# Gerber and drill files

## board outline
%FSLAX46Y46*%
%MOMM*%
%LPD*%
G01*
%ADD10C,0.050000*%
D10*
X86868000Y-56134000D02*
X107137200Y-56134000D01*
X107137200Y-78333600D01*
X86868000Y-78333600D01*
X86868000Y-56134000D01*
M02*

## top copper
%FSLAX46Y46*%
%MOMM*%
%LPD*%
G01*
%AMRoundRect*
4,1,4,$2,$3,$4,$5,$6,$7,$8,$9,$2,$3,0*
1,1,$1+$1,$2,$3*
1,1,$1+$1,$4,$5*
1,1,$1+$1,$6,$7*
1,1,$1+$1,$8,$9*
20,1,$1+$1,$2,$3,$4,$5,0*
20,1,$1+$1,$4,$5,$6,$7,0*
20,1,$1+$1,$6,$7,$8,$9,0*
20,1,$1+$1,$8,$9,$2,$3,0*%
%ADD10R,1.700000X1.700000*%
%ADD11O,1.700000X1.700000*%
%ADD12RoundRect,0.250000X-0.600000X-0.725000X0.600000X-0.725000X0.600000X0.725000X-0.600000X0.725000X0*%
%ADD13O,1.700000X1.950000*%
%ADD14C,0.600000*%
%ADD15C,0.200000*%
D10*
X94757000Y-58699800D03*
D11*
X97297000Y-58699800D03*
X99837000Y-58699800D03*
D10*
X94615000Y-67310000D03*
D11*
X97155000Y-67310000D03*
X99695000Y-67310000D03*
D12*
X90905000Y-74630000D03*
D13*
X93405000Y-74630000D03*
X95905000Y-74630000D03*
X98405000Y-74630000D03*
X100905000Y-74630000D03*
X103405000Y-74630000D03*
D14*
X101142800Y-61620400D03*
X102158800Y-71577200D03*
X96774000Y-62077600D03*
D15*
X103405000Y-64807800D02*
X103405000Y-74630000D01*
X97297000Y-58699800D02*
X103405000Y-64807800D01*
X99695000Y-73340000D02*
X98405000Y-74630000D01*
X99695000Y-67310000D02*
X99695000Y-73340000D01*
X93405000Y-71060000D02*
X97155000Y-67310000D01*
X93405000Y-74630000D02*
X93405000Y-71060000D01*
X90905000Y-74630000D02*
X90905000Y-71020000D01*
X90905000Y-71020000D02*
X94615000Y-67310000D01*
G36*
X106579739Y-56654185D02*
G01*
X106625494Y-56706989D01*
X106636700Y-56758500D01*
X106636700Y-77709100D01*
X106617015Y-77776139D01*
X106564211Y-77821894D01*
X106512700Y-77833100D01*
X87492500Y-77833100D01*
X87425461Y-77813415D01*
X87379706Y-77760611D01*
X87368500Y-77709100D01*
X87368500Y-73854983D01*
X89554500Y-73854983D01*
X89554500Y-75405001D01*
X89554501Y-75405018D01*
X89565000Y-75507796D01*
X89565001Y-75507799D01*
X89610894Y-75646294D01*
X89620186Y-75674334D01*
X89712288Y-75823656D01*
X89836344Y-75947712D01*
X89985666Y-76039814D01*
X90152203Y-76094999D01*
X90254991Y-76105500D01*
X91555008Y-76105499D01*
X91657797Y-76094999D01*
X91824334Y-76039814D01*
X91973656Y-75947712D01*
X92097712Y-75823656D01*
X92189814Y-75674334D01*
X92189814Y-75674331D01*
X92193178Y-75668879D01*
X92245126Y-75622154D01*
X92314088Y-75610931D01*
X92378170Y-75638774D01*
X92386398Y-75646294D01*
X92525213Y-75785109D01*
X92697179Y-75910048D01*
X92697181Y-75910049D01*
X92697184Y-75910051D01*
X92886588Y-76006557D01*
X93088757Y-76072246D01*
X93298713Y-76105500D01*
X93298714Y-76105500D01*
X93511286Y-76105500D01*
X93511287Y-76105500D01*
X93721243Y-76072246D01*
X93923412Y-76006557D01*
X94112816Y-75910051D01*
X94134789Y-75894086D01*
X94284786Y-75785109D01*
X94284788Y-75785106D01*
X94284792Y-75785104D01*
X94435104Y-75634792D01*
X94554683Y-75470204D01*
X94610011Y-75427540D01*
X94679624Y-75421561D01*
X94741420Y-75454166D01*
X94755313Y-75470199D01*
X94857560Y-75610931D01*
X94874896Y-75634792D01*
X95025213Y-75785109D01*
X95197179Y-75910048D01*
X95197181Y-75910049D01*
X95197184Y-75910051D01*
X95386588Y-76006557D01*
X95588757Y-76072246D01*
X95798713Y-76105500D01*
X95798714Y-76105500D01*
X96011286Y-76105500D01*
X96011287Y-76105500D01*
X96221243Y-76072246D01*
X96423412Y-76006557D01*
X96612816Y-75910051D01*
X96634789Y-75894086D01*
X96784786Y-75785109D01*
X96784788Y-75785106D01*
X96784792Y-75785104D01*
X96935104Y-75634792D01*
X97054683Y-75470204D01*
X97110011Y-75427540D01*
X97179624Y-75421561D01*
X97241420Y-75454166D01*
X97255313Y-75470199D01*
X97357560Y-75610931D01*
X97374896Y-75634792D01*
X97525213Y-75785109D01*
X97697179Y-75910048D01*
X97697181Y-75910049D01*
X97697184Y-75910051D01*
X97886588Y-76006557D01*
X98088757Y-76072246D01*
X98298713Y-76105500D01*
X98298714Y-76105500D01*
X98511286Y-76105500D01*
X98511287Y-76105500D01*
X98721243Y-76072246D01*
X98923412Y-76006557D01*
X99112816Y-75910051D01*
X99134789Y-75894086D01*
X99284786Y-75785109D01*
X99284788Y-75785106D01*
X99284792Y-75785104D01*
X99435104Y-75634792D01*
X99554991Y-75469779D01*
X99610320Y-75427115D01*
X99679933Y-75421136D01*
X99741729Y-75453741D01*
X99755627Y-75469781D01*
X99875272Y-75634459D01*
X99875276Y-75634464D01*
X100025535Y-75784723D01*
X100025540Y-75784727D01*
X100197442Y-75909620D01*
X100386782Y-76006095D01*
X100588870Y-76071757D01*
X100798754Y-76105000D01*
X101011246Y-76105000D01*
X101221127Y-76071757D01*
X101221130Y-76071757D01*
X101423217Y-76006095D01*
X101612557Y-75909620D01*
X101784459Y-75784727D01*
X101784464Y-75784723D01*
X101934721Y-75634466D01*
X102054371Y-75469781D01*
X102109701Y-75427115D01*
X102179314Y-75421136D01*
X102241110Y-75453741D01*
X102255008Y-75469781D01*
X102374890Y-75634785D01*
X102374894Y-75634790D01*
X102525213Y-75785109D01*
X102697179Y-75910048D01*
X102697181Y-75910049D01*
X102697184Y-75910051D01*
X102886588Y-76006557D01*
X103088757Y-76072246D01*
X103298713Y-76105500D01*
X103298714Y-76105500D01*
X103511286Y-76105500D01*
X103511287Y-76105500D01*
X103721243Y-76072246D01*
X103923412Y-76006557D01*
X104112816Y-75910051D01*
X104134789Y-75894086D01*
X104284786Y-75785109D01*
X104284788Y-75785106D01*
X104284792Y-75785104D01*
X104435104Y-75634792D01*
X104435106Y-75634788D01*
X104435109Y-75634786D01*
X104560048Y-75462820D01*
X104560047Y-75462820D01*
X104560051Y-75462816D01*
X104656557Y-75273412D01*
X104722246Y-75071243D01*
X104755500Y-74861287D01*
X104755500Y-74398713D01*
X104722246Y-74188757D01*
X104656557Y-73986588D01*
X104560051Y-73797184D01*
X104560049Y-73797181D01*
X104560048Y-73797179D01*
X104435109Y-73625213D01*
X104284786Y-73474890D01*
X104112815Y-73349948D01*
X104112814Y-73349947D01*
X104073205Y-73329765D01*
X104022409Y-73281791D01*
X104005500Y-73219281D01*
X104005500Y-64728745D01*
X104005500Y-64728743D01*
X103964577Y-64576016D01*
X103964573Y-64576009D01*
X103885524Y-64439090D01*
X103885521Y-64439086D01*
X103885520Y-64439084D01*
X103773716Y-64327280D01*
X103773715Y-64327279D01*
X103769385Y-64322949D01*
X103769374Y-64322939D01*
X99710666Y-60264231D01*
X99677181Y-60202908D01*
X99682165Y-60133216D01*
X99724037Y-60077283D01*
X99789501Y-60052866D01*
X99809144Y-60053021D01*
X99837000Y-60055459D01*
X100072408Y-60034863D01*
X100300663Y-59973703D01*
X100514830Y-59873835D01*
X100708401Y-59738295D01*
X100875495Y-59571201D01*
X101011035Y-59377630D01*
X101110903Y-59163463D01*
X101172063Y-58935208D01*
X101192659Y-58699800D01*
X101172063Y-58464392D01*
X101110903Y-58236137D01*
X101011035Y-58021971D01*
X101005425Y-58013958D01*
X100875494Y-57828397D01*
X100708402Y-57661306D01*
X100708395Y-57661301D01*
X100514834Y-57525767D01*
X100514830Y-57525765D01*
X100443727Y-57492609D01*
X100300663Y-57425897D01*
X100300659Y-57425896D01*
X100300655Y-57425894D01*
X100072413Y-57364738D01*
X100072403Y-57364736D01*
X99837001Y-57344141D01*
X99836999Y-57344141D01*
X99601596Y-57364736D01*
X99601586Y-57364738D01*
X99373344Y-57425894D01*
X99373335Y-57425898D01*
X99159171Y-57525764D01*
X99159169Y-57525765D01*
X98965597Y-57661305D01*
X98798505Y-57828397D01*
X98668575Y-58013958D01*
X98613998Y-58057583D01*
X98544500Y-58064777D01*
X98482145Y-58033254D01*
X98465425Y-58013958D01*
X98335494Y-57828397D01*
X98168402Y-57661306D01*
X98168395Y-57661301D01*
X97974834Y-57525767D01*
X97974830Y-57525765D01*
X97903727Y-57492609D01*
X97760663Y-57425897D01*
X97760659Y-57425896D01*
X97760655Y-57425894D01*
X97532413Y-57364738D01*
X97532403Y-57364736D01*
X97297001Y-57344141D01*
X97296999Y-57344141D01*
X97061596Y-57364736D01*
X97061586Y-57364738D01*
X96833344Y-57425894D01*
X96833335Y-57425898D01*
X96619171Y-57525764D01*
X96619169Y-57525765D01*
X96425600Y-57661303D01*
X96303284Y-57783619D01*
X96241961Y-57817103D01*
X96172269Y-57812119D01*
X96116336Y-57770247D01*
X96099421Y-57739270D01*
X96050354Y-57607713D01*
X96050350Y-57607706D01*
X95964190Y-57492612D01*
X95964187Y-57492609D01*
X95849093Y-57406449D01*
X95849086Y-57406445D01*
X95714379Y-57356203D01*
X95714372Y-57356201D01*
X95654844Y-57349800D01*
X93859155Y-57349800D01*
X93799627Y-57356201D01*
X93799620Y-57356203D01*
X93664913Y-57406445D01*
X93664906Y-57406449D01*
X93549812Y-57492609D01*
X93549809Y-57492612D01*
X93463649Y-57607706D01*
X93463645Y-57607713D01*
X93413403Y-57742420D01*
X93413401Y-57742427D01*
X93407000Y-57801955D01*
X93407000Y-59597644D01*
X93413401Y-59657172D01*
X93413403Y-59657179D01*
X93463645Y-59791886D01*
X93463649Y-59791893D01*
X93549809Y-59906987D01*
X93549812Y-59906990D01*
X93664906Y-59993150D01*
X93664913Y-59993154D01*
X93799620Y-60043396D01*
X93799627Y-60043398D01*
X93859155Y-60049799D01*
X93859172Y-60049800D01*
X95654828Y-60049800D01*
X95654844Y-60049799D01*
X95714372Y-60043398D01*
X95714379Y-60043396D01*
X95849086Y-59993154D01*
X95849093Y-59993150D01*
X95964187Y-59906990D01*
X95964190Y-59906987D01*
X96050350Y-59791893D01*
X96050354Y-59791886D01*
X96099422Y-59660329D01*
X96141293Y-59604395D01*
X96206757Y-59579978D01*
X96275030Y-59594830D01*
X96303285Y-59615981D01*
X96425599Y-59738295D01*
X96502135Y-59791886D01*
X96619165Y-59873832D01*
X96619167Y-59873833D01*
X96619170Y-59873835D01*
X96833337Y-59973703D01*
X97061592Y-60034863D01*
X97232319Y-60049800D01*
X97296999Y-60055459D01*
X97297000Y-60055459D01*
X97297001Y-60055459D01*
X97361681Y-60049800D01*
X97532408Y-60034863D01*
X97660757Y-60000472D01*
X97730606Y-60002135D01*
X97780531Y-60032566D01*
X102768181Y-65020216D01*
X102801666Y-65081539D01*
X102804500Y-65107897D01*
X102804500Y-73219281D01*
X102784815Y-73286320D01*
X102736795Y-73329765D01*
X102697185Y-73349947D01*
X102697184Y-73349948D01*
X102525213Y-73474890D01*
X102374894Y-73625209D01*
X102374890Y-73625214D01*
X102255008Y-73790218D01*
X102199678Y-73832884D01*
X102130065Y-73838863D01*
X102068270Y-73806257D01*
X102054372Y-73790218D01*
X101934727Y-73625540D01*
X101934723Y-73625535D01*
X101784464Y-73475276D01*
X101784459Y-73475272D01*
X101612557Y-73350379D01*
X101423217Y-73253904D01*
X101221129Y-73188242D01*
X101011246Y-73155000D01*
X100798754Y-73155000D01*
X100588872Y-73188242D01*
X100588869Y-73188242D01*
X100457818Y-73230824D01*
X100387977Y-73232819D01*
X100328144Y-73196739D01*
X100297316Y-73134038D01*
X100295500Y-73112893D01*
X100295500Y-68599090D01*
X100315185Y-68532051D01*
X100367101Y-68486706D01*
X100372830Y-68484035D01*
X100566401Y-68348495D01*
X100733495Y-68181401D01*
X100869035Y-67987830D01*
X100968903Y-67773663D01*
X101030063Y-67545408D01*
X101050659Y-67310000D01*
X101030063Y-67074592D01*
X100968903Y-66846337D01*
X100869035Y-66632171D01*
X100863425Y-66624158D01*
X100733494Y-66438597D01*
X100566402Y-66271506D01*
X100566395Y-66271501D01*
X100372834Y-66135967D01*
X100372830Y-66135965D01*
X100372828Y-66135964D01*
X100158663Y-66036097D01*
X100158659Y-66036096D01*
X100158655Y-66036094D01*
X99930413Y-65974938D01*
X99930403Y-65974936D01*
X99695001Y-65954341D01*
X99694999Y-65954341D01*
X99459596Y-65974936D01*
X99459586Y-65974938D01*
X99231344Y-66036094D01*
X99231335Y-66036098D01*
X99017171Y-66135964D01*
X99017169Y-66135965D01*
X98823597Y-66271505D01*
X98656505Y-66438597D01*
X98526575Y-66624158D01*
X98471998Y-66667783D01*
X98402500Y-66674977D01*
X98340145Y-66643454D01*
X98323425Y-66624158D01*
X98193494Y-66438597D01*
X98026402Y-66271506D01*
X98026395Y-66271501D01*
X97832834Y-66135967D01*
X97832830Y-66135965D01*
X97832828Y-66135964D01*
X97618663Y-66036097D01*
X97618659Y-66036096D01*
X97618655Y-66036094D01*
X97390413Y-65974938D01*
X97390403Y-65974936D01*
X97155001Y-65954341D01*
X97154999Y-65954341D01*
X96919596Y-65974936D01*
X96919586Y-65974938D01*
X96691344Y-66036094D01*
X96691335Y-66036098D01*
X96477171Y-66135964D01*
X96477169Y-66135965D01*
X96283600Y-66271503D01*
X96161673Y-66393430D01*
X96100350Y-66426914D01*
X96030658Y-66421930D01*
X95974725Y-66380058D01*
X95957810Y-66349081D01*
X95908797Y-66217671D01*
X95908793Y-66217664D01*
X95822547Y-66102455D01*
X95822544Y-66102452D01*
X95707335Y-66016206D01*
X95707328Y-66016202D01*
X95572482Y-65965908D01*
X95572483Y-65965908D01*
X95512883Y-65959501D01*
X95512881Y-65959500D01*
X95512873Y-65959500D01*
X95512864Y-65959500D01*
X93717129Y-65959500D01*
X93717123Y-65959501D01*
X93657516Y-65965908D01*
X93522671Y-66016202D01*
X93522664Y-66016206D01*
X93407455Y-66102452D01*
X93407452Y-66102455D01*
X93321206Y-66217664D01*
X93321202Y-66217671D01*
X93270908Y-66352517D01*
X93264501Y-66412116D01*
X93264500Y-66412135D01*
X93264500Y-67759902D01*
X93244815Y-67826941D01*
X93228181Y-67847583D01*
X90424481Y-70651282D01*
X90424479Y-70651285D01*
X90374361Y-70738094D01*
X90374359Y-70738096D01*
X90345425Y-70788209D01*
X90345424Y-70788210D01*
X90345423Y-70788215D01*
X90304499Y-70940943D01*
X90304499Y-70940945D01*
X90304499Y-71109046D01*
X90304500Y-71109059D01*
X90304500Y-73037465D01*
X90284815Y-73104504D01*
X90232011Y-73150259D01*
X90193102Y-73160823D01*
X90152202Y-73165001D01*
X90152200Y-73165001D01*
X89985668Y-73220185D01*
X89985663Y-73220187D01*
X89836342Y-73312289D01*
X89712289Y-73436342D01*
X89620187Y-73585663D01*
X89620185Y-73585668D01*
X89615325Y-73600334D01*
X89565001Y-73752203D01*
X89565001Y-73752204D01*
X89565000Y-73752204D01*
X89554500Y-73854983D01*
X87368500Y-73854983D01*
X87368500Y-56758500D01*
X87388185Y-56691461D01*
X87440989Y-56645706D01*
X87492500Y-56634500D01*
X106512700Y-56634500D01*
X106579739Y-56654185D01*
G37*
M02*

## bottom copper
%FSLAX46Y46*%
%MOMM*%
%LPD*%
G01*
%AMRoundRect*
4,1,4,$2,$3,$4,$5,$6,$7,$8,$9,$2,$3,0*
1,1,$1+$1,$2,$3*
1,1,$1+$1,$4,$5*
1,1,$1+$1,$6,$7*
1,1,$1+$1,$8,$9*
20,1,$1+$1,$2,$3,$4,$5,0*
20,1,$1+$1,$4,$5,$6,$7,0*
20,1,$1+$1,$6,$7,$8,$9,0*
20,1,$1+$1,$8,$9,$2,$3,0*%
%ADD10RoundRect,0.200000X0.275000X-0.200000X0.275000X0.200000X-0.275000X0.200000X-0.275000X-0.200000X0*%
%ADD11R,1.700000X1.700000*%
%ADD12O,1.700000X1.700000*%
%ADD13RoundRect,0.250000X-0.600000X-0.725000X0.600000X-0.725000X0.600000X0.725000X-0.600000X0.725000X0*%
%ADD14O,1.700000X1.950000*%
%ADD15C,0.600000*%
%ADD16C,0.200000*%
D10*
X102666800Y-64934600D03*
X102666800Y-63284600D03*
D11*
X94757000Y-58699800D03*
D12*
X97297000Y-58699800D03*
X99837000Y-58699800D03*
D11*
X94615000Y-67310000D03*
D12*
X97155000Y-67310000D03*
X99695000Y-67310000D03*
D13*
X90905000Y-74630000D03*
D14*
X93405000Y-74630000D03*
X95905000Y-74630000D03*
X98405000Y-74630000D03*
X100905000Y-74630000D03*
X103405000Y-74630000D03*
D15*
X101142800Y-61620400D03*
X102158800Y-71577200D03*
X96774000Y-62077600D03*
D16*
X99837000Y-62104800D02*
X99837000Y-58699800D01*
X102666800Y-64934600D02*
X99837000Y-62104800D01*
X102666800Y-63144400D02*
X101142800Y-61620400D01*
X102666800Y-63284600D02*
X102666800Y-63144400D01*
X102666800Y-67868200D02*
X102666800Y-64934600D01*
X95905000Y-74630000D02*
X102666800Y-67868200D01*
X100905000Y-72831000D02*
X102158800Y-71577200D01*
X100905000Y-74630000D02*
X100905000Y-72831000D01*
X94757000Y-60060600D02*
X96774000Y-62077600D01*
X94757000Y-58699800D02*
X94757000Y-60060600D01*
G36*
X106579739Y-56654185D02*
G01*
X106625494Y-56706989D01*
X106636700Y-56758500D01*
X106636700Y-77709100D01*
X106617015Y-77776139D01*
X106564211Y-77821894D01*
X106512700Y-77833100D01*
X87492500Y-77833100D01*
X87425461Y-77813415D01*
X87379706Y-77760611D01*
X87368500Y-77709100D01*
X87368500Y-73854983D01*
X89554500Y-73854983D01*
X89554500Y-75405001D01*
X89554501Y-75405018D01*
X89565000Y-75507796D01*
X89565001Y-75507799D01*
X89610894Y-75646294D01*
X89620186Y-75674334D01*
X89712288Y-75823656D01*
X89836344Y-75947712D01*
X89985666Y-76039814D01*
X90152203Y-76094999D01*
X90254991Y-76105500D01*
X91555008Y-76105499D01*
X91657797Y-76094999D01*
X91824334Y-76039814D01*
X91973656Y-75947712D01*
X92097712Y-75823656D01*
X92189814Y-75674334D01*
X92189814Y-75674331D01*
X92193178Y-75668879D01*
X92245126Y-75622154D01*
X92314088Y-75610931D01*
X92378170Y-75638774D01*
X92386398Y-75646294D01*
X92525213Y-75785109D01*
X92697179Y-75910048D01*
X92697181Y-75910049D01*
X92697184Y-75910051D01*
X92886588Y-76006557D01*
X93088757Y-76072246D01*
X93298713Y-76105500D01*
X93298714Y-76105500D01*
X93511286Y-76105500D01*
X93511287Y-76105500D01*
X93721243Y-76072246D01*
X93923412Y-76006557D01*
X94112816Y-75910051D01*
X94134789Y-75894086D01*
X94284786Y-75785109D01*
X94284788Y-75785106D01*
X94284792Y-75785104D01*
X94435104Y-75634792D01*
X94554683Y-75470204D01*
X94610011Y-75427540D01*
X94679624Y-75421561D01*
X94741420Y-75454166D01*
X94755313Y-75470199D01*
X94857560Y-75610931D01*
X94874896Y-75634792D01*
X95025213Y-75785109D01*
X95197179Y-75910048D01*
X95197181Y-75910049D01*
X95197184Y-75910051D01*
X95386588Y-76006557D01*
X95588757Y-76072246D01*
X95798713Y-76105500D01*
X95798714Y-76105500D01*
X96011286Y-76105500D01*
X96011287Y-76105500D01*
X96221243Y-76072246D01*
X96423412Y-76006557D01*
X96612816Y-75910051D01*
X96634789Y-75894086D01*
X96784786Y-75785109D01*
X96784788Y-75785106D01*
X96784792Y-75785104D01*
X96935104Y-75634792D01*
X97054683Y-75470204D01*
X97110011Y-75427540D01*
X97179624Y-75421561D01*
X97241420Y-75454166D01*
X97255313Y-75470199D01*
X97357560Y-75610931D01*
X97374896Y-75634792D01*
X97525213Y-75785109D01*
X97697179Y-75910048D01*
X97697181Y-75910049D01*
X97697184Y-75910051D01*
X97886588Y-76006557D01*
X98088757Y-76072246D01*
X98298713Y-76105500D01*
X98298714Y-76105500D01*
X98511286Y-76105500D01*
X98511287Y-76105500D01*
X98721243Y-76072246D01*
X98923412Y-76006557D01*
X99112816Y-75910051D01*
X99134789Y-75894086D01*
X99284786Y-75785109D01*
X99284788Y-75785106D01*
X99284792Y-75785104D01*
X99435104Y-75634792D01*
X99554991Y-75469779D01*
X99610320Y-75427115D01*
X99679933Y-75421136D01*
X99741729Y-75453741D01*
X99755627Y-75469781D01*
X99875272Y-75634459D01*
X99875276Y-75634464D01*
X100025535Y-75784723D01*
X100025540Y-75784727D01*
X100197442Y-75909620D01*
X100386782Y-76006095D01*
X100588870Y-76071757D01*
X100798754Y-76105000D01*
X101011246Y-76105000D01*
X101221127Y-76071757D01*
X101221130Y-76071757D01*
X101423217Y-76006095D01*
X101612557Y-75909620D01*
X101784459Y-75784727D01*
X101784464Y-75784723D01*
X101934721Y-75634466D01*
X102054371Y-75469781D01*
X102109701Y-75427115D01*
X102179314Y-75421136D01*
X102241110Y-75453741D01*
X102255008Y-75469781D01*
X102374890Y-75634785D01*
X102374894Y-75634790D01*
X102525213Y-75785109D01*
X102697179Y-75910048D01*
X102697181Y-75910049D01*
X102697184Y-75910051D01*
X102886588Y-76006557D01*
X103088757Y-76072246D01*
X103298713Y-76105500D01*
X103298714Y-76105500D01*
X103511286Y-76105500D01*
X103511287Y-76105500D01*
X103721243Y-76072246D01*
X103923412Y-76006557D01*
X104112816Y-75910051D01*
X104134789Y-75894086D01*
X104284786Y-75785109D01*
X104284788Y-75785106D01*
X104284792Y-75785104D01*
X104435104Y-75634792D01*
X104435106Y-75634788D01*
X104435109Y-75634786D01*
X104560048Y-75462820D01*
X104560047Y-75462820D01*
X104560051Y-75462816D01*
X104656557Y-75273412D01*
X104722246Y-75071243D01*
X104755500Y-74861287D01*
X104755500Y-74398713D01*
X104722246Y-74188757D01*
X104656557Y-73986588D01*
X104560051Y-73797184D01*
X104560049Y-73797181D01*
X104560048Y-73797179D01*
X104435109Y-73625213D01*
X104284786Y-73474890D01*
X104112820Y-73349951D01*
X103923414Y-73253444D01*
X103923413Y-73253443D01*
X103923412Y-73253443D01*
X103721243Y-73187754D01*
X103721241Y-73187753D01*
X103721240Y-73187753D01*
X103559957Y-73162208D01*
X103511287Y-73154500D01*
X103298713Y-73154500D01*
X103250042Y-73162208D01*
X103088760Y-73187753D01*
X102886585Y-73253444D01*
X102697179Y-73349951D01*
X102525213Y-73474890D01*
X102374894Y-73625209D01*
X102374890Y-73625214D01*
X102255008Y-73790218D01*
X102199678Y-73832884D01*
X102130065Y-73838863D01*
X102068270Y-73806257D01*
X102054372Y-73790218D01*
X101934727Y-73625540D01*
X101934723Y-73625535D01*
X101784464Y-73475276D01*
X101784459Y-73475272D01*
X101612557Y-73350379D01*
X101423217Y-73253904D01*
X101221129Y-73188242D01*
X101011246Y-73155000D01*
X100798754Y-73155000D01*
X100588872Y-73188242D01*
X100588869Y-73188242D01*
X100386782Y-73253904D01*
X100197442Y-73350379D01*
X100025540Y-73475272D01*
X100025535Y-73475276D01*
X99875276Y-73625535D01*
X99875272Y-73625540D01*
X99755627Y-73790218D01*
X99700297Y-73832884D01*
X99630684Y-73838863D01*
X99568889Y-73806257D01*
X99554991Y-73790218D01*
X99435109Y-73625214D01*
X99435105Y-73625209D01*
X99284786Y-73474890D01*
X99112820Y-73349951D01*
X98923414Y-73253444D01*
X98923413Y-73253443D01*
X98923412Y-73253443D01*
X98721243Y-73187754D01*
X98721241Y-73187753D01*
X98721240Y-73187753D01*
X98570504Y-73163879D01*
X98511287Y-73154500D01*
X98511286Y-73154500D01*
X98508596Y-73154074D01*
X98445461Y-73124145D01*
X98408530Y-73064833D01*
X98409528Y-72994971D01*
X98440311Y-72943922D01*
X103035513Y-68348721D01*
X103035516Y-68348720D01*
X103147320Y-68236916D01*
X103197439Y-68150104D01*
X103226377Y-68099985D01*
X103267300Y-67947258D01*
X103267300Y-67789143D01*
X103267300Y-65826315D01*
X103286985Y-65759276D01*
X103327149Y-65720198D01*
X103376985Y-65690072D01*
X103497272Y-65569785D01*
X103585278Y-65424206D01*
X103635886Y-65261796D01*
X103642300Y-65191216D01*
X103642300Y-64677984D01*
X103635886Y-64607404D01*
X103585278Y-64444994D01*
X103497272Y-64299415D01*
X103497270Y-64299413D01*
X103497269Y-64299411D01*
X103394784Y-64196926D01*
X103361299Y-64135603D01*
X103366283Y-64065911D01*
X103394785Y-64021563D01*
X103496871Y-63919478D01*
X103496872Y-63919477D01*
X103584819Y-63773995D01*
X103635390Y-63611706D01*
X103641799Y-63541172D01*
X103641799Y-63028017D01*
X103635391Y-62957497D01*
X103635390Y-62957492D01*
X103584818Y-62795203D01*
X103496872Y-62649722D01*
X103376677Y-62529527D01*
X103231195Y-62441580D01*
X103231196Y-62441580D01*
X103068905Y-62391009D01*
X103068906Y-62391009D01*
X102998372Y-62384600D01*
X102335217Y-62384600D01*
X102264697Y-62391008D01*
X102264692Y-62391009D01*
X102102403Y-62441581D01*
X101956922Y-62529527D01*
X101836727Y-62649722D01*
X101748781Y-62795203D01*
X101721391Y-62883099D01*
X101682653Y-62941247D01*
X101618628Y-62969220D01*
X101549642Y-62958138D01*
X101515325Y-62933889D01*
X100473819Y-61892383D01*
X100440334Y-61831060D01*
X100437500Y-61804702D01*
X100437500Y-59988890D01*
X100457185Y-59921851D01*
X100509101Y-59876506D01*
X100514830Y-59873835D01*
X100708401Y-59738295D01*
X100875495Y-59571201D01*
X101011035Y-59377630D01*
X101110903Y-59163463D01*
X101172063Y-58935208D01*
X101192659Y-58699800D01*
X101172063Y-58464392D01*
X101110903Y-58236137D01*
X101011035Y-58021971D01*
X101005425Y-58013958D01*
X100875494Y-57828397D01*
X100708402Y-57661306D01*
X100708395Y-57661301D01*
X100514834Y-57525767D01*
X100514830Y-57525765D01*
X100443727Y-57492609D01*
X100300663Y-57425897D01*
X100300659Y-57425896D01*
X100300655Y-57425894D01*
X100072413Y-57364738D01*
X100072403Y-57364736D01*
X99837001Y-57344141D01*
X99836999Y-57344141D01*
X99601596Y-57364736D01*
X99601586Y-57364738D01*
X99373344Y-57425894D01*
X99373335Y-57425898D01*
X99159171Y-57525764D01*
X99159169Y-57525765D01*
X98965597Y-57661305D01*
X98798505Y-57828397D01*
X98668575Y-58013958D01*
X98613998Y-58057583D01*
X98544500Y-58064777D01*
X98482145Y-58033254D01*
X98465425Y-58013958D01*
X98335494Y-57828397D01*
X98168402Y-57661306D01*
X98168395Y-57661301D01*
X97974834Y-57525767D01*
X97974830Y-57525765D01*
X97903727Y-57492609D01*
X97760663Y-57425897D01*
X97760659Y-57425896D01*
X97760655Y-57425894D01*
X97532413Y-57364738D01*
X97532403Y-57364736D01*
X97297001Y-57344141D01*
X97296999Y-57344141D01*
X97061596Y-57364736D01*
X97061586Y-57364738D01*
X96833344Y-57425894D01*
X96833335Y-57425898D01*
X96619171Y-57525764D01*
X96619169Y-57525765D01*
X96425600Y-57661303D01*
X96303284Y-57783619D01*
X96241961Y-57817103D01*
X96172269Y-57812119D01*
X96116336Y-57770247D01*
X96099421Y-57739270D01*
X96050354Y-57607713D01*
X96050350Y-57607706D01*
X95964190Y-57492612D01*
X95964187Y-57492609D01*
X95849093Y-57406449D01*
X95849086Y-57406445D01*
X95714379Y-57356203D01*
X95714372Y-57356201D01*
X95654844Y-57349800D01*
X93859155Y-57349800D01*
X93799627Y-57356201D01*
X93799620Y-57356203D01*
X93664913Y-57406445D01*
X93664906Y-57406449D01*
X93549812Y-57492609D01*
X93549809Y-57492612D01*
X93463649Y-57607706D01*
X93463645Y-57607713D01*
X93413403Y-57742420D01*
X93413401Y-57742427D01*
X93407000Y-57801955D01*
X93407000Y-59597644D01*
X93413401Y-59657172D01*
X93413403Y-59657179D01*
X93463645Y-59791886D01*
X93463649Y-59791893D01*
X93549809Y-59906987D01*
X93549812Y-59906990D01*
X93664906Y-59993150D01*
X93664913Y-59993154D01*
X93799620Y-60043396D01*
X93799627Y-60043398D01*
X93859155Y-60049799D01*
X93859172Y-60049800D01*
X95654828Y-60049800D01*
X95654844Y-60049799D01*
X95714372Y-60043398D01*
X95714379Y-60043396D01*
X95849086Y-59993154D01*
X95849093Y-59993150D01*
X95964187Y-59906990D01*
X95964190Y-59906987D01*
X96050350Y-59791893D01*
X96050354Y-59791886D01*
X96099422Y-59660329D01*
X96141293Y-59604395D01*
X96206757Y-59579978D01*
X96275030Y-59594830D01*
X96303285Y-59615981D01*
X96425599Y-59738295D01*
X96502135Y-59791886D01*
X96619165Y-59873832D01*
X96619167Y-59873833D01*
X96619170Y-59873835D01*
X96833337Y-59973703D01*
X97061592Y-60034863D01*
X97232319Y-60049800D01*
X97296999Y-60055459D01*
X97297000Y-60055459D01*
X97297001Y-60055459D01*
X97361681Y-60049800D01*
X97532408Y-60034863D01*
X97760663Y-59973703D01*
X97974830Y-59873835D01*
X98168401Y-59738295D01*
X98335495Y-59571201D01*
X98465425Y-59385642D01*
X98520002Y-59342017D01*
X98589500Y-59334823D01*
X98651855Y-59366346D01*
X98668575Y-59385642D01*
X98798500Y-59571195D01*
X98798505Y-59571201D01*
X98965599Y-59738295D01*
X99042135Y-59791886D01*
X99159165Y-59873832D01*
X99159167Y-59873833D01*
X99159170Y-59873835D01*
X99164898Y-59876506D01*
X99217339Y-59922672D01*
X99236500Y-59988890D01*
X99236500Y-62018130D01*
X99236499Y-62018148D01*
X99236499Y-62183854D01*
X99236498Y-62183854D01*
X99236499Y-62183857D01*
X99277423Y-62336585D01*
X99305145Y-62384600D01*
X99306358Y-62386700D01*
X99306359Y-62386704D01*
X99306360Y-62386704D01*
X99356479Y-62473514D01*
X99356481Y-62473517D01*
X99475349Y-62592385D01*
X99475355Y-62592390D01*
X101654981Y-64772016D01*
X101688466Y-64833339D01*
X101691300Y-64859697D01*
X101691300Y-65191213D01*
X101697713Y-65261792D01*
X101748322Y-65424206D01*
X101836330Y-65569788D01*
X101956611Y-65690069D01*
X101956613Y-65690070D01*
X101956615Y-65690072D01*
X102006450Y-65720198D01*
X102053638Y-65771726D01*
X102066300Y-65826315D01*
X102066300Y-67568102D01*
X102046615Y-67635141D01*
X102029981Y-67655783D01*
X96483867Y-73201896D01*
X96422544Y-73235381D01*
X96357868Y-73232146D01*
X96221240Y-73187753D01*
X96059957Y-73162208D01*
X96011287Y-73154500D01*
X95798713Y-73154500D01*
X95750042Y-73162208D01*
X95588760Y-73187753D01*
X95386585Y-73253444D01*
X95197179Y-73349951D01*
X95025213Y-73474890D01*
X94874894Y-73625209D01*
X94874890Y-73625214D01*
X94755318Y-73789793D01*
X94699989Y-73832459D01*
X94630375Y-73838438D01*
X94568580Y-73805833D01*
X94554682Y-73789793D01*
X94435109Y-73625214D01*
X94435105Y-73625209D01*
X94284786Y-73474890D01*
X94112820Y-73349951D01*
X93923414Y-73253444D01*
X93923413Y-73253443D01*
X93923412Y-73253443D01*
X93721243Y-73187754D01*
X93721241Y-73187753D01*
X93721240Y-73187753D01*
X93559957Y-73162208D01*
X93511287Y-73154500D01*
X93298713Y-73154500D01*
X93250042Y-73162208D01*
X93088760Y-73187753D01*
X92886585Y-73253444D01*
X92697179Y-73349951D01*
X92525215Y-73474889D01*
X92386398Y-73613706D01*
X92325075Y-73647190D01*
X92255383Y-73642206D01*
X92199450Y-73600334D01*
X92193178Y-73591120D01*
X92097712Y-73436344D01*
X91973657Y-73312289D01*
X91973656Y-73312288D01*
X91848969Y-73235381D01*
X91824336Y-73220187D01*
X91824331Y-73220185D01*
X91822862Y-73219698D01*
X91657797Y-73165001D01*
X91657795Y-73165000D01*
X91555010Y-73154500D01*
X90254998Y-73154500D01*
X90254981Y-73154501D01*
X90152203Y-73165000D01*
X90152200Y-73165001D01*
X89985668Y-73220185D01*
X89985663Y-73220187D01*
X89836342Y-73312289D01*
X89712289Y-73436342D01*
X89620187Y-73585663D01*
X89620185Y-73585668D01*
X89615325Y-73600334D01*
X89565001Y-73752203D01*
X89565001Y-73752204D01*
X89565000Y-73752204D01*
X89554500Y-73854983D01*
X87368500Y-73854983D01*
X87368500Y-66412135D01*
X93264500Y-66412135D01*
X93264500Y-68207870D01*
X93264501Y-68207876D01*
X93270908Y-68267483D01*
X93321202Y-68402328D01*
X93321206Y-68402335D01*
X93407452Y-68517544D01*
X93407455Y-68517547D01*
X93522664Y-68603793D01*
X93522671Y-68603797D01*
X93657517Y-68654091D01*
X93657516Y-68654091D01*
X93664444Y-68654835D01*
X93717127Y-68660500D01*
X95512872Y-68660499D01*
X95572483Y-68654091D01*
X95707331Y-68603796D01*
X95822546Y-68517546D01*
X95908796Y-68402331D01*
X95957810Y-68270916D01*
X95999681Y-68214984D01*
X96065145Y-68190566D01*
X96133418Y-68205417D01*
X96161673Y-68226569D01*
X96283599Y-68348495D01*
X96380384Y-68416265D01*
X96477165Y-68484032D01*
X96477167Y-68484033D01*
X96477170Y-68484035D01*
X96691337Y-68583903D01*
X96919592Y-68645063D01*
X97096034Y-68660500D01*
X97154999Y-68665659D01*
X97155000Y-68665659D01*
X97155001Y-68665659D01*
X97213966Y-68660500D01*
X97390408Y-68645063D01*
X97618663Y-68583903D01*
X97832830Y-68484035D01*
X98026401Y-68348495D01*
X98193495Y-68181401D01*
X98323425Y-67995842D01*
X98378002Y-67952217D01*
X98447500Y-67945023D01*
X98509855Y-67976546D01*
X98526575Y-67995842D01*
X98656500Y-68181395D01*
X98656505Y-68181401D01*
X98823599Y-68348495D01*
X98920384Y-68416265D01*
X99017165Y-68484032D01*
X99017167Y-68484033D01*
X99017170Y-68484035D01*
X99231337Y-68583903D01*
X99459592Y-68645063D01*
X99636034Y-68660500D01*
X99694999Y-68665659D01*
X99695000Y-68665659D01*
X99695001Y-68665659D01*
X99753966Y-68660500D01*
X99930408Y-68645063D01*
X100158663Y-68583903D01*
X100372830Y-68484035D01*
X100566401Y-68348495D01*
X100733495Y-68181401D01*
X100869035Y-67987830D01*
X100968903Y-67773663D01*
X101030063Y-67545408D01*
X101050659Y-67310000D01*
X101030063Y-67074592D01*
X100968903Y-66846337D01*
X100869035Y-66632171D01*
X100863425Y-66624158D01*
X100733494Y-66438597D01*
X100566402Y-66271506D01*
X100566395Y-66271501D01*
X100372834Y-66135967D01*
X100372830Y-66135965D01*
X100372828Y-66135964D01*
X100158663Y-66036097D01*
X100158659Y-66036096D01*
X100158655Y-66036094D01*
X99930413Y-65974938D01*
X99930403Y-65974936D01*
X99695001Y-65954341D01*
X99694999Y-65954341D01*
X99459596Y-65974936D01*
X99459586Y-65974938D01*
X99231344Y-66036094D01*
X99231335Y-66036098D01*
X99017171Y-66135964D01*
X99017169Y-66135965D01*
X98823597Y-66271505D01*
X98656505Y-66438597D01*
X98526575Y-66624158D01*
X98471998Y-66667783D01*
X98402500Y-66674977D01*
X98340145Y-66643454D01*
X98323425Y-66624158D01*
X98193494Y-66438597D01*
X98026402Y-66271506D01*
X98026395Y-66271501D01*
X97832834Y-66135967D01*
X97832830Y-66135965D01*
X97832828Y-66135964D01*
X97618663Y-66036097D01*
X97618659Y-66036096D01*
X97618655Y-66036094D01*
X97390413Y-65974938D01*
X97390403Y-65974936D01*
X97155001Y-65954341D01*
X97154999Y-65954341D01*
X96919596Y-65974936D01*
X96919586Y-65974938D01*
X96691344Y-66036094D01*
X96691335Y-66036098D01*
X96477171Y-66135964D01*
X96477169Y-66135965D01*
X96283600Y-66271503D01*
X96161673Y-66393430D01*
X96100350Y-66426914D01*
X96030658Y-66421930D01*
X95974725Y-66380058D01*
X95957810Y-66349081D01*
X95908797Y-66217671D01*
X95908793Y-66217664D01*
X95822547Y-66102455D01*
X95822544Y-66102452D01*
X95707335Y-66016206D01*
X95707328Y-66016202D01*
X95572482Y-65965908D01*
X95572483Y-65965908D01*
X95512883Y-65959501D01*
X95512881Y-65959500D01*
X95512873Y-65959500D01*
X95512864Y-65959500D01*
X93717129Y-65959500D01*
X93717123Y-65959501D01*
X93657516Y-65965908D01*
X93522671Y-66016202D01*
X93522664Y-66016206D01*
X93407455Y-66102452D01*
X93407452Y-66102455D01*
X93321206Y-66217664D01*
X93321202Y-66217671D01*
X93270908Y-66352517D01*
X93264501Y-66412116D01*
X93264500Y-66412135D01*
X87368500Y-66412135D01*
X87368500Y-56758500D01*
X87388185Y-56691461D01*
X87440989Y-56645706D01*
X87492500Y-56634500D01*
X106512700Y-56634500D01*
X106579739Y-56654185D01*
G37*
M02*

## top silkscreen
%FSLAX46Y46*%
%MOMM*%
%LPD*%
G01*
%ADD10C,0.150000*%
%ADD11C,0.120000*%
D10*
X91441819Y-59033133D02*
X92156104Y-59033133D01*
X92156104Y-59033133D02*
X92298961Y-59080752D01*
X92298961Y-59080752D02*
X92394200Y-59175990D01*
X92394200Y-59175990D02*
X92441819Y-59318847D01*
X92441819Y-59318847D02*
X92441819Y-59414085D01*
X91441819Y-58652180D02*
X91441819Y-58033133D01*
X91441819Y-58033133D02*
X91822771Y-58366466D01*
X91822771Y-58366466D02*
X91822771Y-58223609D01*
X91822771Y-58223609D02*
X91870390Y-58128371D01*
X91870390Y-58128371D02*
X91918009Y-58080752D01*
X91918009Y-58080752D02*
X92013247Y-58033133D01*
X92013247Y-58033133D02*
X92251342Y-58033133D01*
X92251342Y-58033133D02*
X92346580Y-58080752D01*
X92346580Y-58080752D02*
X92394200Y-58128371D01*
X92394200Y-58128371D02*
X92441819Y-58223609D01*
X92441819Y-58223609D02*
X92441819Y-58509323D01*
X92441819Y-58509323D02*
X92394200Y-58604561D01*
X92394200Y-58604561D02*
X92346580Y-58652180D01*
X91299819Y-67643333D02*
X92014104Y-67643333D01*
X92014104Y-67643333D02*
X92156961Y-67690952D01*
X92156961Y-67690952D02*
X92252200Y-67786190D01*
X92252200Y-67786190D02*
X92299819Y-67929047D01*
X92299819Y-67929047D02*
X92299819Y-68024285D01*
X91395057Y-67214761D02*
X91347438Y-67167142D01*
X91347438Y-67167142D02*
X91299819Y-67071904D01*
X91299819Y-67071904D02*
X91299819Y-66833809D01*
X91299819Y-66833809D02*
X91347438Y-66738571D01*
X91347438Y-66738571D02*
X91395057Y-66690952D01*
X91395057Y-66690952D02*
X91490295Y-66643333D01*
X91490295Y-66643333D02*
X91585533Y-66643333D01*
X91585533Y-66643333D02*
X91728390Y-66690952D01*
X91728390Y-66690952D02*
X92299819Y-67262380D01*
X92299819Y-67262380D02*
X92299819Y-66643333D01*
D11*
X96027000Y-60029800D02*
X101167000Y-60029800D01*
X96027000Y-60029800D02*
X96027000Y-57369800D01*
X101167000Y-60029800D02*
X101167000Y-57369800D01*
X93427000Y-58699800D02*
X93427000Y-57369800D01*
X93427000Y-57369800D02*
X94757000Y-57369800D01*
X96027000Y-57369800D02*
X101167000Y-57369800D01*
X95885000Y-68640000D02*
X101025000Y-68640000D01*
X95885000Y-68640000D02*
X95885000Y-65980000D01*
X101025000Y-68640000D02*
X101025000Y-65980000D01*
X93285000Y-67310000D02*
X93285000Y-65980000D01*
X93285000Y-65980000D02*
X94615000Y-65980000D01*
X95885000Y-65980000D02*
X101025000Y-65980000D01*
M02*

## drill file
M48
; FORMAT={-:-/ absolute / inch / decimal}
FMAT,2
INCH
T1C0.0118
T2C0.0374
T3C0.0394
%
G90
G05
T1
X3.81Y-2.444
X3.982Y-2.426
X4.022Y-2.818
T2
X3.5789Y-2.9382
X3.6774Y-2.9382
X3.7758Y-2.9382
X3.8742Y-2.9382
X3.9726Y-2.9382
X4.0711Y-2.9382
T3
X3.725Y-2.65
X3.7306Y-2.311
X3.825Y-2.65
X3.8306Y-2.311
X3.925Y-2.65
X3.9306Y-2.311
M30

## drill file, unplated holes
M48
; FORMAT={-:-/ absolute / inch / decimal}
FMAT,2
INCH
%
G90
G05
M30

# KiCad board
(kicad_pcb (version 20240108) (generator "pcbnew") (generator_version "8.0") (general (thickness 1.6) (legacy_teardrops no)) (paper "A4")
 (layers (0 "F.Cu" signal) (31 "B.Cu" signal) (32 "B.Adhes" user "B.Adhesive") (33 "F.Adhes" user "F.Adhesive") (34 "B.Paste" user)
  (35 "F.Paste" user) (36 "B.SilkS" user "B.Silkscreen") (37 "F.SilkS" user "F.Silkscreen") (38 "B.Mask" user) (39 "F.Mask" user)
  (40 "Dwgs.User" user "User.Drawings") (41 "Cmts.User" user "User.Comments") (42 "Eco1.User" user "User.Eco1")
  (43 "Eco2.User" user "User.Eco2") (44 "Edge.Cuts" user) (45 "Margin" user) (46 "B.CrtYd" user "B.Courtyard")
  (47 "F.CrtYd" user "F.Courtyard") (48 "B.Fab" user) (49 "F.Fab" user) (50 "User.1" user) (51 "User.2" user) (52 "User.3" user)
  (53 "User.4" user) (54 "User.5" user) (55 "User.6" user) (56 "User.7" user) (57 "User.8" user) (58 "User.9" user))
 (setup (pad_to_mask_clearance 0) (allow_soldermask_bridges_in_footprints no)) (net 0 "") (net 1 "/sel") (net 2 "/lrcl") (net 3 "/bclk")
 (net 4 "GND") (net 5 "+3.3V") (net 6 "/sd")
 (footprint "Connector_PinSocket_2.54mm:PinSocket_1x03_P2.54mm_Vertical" (layer "F.Cu") (at 94.615 67.31 90)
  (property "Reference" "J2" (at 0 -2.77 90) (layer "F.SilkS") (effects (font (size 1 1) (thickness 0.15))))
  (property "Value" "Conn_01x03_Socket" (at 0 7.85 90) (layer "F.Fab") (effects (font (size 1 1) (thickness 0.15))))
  (fp_line (start 1.33 -1.33) (end 1.33 0) (stroke (width 0.12) (type solid)) (layer "F.SilkS"))
  (fp_line (start 0 -1.33) (end 1.33 -1.33) (stroke (width 0.12) (type solid)) (layer "F.SilkS"))
  (fp_line (start 1.33 1.27) (end 1.33 6.41) (stroke (width 0.12) (type solid)) (layer "F.SilkS"))
  (fp_line (start -1.33 1.27) (end 1.33 1.27) (stroke (width 0.12) (type solid)) (layer "F.SilkS"))
  (fp_line (start -1.33 1.27) (end -1.33 6.41) (stroke (width 0.12) (type solid)) (layer "F.SilkS"))
  (fp_line (start -1.33 6.41) (end 1.33 6.41) (stroke (width 0.12) (type solid)) (layer "F.SilkS"))
  (pad "1" thru_hole rect (at 0 0 90) (size 1.7 1.7) (drill 1) (layers "*.Cu" "*.Mask") (remove_unused_layers no) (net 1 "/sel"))
  (pad "2" thru_hole oval (at 0 2.54 90) (size 1.7 1.7) (drill 1) (layers "*.Cu" "*.Mask") (remove_unused_layers no) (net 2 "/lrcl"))
  (pad "3" thru_hole oval (at 0 5.08 90) (size 1.7 1.7) (drill 1) (layers "*.Cu" "*.Mask") (remove_unused_layers no) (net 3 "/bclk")))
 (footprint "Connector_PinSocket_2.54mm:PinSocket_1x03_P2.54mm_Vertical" (layer "F.Cu") (at 94.757 58.6998 90)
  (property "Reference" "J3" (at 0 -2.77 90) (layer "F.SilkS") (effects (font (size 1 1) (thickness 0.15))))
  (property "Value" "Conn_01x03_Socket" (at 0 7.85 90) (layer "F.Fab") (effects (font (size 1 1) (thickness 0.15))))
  (fp_line (start 1.33 -1.33) (end 1.33 0) (stroke (width 0.12) (type solid)) (layer "F.SilkS"))
  (fp_line (start 0 -1.33) (end 1.33 -1.33) (stroke (width 0.12) (type solid)) (layer "F.SilkS"))
  (fp_line (start 1.33 1.27) (end 1.33 6.41) (stroke (width 0.12) (type solid)) (layer "F.SilkS"))
  (fp_line (start -1.33 1.27) (end 1.33 1.27) (stroke (width 0.12) (type solid)) (layer "F.SilkS"))
  (fp_line (start -1.33 1.27) (end -1.33 6.41) (stroke (width 0.12) (type solid)) (layer "F.SilkS"))
  (fp_line (start -1.33 6.41) (end 1.33 6.41) (stroke (width 0.12) (type solid)) (layer "F.SilkS"))
  (pad "1" thru_hole rect (at 0 0 90) (size 1.7 1.7) (drill 1) (layers "*.Cu" "*.Mask") (remove_unused_layers no) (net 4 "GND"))
  (pad "2" thru_hole oval (at 0 2.54 90) (size 1.7 1.7) (drill 1) (layers "*.Cu" "*.Mask") (remove_unused_layers no) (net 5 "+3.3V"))
  (pad "3" thru_hole oval (at 0 5.08 90) (size 1.7 1.7) (drill 1) (layers "*.Cu" "*.Mask") (remove_unused_layers no) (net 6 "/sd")))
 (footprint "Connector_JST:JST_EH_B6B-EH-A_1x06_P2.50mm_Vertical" (layer "B.Cu") (at 90.905 74.63)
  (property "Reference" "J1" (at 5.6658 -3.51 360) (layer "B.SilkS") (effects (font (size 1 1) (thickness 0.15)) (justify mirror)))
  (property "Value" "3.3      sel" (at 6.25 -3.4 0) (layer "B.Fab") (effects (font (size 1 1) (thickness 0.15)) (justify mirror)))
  (pad "1" thru_hole roundrect (at 0 0) (size 1.7 1.95) (drill 0.95) (layers "*.Cu" "*.Mask") (remove_unused_layers no)
   (roundrect_rratio 0.147059) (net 1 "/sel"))
  (pad "2" thru_hole oval (at 2.5 0) (size 1.7 1.95) (drill 0.95) (layers "*.Cu" "*.Mask") (remove_unused_layers no) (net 2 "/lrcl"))
  (pad "3" thru_hole oval (at 5 0) (size 1.7 1.95) (drill 0.95) (layers "*.Cu" "*.Mask") (remove_unused_layers no) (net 6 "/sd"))
  (pad "4" thru_hole oval (at 7.5 0) (size 1.7 1.95) (drill 0.95) (layers "*.Cu" "*.Mask") (remove_unused_layers no) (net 3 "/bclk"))
  (pad "5" thru_hole oval (at 10 0) (size 1.7 1.95) (drill 0.95) (layers "*.Cu" "*.Mask") (remove_unused_layers no) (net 4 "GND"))
  (pad "6" thru_hole oval (at 12.5 0) (size 1.7 1.95) (drill 0.95) (layers "*.Cu" "*.Mask") (remove_unused_layers no) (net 5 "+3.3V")))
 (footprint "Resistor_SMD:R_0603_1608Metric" (layer "B.Cu") (at 102.6668 64.1096 90)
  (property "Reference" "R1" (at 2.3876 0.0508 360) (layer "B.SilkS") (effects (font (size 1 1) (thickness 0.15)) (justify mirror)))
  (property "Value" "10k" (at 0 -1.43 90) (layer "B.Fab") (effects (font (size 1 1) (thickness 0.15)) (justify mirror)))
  (pad "1" smd roundrect (at -0.825 0 90) (size 0.8 0.95) (layers "B.Cu" "B.Paste" "B.Mask") (roundrect_rratio 0.25) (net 6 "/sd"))
  (pad "2" smd roundrect (at 0.825 0 90) (size 0.8 0.95) (layers "B.Cu" "B.Paste" "B.Mask") (roundrect_rratio 0.25) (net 4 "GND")))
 (gr_rect (start 86.868 56.134) (end 107.1372 78.3336) (stroke (width 0.05) (type default)) (fill none) (layer "Edge.Cuts"))
 (segment (start 90.905 74.63) (end 90.905 71.02) (width 0.2) (layer "F.Cu") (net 1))
 (segment (start 90.905 71.02) (end 94.615 67.31) (width 0.2) (layer "F.Cu") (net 1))
 (segment (start 102.6668 67.8682) (end 102.6668 64.9346) (width 0.2) (layer "B.Cu") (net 6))
 (segment (start 95.905 74.63) (end 102.6668 67.8682) (width 0.2) (layer "B.Cu") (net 6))
 (segment (start 99.837 62.1048) (end 99.837 58.6998) (width 0.2) (layer "B.Cu") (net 6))
 (segment (start 102.6668 64.9346) (end 99.837 62.1048) (width 0.2) (layer "B.Cu") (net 6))
 (segment (start 103.405 64.8078) (end 103.405 74.63) (width 0.2) (layer "F.Cu") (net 5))
 (segment (start 97.297 58.6998) (end 103.405 64.8078) (width 0.2) (layer "F.Cu") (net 5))
 (via (at 96.774 62.0776) (size 0.6) (drill 0.3) (layers "F.Cu" "B.Cu") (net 4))
 (via (at 102.1588 71.5772) (size 0.6) (drill 0.3) (layers "F.Cu" "B.Cu") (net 4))
 (via (at 101.1428 61.6204) (size 0.6) (drill 0.3) (layers "F.Cu" "B.Cu") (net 4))
 (segment (start 102.6668 63.2846) (end 102.6668 63.1444) (width 0.2) (layer "B.Cu") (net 4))
 (segment (start 100.905 74.63) (end 100.905 72.831) (width 0.2) (layer "B.Cu") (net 4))
 (segment (start 100.905 72.831) (end 102.1588 71.5772) (width 0.2) (layer "B.Cu") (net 4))
 (segment (start 94.757 58.6998) (end 94.757 60.0606) (width 0.2) (layer "B.Cu") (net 4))
 (segment (start 94.757 60.0606) (end 96.774 62.0776) (width 0.2) (layer "B.Cu") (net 4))
 (segment (start 102.6668 63.1444) (end 101.1428 61.6204) (width 0.2) (layer "B.Cu") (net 4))
 (segment (start 99.695 67.31) (end 99.695 73.34) (width 0.2) (layer "F.Cu") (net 3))
 (segment (start 99.695 73.34) (end 98.405 74.63) (width 0.2) (layer "F.Cu") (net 3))
 (segment (start 93.405 74.63) (end 93.405 71.06) (width 0.2) (layer "F.Cu") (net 2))
 (segment (start 93.405 71.06) (end 97.155 67.31) (width 0.2) (layer "F.Cu") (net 2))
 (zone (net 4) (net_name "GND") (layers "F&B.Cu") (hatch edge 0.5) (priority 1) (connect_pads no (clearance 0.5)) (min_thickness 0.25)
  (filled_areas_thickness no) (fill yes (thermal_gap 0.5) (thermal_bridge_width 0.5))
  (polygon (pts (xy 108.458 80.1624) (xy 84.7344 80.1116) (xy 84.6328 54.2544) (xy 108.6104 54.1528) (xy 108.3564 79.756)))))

